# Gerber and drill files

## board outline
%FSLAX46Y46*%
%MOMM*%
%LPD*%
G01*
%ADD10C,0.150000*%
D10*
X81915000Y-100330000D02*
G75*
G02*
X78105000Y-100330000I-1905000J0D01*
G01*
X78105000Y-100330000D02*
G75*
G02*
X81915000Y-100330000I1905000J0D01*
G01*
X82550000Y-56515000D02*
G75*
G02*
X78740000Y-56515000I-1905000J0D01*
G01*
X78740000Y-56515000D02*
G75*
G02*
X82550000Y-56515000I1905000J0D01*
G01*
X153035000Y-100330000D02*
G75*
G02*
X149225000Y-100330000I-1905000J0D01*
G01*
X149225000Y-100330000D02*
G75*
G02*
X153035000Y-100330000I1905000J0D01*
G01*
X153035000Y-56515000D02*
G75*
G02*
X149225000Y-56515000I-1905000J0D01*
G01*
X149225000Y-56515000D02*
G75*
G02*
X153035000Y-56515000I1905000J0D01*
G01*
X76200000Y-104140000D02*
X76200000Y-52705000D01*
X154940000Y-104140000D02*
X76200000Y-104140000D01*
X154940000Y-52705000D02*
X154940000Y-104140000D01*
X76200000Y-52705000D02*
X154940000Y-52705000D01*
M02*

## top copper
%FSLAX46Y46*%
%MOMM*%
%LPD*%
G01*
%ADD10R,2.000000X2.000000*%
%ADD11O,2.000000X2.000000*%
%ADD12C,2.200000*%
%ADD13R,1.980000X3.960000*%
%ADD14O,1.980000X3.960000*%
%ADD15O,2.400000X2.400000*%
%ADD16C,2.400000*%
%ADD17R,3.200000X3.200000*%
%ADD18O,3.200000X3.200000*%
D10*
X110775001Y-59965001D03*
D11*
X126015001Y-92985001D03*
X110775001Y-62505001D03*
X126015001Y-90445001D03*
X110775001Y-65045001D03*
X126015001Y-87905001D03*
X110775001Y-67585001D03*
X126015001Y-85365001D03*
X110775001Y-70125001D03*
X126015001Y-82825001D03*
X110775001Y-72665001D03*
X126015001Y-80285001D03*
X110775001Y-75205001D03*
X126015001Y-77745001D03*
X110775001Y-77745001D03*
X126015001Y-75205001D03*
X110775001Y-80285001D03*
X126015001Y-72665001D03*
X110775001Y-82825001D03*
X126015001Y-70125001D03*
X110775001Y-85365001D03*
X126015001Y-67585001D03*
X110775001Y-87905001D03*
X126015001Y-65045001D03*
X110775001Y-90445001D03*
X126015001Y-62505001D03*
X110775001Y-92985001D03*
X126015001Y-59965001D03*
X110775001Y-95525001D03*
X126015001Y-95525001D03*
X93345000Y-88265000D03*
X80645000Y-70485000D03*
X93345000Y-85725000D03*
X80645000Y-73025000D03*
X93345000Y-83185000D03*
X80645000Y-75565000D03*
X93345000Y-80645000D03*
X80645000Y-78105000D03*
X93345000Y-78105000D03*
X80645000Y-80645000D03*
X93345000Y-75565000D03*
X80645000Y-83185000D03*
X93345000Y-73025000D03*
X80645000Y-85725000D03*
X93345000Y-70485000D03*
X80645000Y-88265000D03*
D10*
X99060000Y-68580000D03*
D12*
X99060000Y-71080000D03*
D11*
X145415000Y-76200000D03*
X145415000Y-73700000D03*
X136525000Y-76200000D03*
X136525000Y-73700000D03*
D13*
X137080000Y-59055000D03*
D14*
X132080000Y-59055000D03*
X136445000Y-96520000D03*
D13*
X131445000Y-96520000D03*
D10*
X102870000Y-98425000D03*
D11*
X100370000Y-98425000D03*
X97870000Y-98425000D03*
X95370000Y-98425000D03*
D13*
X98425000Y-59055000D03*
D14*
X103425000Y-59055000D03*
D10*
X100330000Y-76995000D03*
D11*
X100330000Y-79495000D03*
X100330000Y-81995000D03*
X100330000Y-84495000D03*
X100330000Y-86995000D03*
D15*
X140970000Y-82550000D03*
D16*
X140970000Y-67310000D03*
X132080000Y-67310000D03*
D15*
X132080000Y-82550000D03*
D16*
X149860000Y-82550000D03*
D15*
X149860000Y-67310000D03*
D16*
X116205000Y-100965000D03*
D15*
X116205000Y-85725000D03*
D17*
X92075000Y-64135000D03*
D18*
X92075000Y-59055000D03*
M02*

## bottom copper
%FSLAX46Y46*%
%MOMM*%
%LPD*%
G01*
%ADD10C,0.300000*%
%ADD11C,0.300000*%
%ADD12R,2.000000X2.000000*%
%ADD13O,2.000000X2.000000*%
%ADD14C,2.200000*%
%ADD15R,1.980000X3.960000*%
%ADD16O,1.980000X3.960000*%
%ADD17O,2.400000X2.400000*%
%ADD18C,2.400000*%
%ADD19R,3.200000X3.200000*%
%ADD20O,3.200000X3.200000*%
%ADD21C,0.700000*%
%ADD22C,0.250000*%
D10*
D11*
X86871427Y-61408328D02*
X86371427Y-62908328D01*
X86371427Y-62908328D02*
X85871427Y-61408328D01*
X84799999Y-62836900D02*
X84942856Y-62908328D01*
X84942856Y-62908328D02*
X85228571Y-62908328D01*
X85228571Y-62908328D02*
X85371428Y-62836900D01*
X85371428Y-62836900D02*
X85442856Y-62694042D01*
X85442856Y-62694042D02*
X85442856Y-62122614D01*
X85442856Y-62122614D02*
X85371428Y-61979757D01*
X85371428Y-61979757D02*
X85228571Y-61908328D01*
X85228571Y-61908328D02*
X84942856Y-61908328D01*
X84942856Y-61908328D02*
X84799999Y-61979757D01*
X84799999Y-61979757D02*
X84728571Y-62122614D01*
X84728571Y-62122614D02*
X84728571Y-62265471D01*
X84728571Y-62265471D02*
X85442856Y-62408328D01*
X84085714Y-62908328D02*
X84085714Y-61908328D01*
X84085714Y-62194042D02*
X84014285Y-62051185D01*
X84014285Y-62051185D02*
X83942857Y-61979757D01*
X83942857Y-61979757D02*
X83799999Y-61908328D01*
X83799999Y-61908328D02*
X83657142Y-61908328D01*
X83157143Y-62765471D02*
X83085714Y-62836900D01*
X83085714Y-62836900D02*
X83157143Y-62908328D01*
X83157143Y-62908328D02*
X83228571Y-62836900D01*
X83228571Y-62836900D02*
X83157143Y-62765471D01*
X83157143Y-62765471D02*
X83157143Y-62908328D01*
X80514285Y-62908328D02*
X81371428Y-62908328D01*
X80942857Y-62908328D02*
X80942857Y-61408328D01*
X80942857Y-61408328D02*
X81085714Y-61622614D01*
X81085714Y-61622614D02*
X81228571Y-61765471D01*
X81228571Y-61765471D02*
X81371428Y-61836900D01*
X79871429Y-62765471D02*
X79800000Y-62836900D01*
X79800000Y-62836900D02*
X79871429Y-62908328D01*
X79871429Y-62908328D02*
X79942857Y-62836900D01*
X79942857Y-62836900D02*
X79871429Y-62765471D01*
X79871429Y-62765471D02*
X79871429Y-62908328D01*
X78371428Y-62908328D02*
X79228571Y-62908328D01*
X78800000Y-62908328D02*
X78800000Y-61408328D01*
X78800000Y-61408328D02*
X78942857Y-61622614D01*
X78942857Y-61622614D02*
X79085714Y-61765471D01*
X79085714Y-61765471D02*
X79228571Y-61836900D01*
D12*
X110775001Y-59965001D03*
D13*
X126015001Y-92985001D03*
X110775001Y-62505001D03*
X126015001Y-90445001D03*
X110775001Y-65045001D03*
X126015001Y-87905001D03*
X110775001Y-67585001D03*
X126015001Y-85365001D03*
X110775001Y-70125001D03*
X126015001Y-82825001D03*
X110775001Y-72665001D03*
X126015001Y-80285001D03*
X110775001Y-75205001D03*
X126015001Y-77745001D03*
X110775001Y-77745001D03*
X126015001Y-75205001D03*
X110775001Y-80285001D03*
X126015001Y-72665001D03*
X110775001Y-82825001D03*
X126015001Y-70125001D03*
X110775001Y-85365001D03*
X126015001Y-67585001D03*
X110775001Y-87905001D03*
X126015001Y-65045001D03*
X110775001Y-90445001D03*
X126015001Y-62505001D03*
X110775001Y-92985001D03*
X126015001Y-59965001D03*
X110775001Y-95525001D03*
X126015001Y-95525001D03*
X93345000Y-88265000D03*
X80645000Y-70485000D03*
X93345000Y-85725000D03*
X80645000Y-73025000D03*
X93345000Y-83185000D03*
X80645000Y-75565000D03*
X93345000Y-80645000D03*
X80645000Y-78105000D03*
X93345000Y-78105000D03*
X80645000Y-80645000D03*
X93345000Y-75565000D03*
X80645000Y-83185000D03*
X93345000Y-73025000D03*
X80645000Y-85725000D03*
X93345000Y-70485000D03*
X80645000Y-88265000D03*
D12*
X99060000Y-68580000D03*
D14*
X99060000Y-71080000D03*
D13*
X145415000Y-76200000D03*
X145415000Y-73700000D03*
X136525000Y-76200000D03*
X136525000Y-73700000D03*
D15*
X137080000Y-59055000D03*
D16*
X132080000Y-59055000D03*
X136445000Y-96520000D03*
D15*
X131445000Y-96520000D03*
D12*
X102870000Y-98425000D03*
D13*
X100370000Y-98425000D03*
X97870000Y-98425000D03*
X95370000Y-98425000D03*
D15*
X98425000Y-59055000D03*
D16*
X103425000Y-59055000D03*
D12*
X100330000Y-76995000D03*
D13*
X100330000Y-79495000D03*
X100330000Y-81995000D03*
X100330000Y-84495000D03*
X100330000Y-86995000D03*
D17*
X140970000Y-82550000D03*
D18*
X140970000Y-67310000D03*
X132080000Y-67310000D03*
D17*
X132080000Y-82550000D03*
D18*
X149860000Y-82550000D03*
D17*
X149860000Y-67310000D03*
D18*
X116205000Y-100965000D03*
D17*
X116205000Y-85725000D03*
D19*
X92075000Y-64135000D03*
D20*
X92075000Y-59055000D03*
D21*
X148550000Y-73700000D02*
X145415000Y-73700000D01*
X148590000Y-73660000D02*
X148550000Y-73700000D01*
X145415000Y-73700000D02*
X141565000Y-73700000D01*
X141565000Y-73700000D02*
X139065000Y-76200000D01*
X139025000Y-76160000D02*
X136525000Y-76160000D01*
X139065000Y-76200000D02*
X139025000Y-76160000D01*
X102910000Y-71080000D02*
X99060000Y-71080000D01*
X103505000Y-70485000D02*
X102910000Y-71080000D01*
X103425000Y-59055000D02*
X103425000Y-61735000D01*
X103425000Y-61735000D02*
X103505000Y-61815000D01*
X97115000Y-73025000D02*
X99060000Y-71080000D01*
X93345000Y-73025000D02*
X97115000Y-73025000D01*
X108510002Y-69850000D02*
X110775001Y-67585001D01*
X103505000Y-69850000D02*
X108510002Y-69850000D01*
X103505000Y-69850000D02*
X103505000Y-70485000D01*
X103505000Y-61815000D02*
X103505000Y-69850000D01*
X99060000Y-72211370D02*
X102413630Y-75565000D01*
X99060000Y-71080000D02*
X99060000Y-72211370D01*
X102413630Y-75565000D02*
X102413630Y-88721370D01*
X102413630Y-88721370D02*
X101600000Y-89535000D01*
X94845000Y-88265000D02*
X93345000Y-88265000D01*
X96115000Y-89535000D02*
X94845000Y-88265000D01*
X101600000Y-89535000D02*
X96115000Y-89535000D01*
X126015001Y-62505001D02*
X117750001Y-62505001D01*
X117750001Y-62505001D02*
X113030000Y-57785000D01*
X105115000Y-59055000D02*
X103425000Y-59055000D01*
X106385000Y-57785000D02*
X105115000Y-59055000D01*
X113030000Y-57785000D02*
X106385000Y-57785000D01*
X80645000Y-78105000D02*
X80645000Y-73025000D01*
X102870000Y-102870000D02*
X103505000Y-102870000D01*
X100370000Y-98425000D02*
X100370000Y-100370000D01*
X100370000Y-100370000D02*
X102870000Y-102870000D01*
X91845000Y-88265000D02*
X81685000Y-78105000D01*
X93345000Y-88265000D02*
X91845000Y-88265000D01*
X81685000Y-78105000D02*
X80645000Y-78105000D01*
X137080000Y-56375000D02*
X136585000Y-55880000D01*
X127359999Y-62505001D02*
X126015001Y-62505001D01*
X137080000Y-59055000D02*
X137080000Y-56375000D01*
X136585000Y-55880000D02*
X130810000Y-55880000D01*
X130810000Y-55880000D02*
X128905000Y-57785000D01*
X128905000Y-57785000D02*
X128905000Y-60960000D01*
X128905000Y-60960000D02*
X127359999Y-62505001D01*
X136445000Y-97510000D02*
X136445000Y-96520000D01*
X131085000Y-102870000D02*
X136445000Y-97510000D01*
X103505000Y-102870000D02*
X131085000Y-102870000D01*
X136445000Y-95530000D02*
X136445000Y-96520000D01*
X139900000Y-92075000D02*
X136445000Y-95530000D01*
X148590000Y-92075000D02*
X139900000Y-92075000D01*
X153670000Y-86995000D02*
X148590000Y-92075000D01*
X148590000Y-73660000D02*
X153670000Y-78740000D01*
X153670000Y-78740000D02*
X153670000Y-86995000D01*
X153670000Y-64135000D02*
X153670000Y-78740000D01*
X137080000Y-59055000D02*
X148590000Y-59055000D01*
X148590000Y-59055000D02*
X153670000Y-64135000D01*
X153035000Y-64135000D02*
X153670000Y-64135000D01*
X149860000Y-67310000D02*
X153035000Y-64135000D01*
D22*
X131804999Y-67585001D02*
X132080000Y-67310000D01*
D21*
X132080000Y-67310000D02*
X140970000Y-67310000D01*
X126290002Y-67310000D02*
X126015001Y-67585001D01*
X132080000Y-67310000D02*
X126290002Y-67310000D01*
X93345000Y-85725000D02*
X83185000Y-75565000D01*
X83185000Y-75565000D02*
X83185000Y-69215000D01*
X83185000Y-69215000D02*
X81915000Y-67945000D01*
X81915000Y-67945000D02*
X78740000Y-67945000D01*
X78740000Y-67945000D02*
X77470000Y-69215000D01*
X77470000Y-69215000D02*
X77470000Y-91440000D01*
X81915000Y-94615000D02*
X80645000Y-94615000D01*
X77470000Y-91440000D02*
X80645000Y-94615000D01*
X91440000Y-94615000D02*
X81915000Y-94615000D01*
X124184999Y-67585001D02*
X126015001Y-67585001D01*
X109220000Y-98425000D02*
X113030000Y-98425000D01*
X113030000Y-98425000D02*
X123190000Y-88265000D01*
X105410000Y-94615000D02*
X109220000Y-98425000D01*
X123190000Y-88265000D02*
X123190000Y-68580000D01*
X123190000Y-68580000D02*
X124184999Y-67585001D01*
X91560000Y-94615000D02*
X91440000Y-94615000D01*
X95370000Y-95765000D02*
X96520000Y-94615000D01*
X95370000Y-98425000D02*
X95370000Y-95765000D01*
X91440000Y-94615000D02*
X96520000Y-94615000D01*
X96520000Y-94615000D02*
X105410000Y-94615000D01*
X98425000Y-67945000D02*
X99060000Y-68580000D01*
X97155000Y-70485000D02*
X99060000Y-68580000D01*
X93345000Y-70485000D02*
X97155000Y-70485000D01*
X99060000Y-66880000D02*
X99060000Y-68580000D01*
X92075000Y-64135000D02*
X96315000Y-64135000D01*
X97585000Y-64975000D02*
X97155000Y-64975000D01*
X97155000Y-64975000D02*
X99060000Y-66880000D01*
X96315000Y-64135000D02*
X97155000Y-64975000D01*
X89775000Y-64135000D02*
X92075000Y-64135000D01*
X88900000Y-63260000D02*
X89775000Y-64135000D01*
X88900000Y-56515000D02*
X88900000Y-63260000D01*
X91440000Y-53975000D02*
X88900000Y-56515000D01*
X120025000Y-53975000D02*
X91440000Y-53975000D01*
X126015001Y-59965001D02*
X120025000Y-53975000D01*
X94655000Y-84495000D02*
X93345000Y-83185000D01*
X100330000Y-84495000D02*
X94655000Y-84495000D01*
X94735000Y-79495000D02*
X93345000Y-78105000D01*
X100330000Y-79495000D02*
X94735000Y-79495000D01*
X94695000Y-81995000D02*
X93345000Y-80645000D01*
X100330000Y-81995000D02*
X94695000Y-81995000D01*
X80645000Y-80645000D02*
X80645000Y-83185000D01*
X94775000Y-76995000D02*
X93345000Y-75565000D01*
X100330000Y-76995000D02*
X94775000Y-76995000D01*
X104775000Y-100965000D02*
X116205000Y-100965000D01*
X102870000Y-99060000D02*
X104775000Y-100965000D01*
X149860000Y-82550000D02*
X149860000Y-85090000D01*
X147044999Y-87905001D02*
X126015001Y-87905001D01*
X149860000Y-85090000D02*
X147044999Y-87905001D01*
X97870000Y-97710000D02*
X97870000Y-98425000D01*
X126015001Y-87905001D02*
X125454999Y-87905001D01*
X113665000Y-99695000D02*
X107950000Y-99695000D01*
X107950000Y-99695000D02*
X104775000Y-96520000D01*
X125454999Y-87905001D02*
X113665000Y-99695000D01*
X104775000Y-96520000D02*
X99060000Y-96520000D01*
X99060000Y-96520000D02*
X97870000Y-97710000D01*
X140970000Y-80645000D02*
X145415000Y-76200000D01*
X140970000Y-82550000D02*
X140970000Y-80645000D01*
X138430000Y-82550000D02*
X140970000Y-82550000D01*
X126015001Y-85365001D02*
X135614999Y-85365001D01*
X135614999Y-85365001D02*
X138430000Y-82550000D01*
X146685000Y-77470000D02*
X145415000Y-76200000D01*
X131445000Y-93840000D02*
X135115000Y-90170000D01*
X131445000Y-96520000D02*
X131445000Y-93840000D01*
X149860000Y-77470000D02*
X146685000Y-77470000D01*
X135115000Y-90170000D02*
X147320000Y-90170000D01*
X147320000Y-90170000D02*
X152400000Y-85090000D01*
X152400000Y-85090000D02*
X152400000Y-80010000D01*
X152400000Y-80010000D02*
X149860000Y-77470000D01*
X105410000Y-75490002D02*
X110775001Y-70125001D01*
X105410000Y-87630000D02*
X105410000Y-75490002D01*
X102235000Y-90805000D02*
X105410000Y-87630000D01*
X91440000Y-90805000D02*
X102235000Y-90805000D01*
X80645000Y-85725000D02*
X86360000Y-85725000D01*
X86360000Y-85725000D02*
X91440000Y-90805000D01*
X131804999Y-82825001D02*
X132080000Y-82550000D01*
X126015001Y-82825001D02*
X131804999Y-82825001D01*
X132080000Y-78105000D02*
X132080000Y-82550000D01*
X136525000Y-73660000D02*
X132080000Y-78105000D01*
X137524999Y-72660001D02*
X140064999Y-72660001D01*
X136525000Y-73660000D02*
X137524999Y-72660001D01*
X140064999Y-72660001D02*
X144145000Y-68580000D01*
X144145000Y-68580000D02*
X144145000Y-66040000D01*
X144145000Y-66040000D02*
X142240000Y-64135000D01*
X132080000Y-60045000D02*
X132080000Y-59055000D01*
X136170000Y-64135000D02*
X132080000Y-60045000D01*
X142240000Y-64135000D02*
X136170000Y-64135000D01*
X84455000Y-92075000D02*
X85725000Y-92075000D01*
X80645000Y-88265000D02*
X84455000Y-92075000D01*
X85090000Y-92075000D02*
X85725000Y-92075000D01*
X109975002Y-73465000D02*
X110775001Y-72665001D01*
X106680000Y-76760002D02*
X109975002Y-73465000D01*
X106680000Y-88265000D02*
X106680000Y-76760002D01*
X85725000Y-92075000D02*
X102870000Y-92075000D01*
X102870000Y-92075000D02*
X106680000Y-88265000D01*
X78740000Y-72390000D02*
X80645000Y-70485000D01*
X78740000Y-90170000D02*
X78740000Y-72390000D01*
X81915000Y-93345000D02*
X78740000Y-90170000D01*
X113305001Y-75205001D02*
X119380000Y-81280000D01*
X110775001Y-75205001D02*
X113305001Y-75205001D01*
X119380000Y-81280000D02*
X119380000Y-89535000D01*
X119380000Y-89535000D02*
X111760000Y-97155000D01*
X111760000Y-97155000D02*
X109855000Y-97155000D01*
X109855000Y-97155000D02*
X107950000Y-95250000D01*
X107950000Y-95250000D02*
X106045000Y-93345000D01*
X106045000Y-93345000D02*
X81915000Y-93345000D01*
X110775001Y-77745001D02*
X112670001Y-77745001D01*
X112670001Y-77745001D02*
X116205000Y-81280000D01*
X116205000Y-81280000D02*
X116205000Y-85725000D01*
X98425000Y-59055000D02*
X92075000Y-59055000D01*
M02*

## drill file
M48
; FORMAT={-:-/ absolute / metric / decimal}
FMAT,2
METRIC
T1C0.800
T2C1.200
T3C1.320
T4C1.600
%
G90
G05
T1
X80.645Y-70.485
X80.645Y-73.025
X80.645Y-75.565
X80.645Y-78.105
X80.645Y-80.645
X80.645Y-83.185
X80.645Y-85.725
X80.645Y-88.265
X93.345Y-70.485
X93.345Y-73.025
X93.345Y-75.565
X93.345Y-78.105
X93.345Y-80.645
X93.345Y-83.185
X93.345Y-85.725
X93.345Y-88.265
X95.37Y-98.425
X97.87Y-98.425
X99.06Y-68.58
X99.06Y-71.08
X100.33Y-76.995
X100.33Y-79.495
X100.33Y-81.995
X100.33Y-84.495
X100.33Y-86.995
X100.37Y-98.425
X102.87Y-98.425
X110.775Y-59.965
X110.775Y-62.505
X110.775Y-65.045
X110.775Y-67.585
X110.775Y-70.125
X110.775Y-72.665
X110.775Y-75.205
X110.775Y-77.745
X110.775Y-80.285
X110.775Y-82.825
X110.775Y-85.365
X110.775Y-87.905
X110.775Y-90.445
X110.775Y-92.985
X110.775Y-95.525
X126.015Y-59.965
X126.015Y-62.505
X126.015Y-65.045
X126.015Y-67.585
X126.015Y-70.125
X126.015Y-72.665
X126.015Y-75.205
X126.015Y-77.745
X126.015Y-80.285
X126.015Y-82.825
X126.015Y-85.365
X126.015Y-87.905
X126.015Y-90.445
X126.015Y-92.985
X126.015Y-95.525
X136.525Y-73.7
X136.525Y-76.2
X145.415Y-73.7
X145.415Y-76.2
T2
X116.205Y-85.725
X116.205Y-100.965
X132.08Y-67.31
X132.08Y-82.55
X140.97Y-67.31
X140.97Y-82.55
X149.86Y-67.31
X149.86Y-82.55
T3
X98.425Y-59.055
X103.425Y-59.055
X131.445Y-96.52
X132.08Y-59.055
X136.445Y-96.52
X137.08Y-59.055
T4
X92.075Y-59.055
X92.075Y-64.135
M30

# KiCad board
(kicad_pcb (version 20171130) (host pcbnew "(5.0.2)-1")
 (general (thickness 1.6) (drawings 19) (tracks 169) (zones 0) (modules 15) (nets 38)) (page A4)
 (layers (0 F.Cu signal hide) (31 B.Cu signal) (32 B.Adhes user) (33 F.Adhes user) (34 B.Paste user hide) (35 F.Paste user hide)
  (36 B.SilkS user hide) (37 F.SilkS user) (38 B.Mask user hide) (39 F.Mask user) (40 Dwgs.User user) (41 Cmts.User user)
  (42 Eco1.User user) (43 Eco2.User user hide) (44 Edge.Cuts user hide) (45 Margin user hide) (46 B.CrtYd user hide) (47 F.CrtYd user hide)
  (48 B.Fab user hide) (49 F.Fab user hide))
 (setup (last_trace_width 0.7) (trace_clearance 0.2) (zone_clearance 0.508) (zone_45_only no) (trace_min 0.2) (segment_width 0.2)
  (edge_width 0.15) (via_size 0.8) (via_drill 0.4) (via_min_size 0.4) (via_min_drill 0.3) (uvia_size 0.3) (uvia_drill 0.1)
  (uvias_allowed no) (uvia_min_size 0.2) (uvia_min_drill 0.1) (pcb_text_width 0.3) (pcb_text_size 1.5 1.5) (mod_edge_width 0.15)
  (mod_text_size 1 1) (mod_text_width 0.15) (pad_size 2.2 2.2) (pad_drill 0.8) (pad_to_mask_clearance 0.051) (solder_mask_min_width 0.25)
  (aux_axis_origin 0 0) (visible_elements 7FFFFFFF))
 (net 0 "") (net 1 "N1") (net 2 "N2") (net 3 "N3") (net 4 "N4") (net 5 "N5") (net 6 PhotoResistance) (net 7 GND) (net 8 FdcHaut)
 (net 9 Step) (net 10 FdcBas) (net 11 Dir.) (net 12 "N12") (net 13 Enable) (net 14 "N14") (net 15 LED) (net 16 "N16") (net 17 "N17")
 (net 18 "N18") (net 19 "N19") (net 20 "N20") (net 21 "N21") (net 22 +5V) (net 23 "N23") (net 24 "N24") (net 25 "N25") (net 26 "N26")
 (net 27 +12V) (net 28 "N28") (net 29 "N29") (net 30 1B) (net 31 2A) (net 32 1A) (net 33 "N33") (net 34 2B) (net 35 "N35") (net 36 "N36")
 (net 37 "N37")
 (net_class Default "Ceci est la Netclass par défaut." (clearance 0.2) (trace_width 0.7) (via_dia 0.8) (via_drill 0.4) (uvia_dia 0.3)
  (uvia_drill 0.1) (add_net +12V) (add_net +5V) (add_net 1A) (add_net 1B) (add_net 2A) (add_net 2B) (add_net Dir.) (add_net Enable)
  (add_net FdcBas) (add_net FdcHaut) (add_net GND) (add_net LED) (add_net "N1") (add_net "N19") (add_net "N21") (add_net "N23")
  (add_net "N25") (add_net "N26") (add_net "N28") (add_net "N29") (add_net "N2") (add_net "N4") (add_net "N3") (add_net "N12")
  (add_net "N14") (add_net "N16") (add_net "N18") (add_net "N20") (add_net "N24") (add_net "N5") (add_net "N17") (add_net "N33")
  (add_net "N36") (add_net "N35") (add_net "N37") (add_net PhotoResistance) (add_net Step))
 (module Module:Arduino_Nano (layer F.Cu) (at 110.775001 59.965001)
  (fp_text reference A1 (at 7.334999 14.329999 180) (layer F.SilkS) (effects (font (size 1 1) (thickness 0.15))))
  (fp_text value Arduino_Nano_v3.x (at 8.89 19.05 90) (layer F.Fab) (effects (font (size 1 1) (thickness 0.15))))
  (pad 1 thru_hole rect (at 0 0) (size 2 2) (drill 0.8) (layers *.Cu *.Mask) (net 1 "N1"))
  (pad 17 thru_hole oval (at 15.24 33.02) (size 2 2) (drill 0.8) (layers *.Cu *.Mask) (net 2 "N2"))
  (pad 2 thru_hole oval (at 0 2.54) (size 2 2) (drill 0.8) (layers *.Cu *.Mask) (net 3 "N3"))
  (pad 18 thru_hole oval (at 15.24 30.48) (size 2 2) (drill 0.8) (layers *.Cu *.Mask) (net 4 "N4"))
  (pad 3 thru_hole oval (at 0 5.08) (size 2 2) (drill 0.8) (layers *.Cu *.Mask) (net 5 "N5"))
  (pad 19 thru_hole oval (at 15.24 27.94) (size 2 2) (drill 0.8) (layers *.Cu *.Mask) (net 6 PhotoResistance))
  (pad 4 thru_hole oval (at 0 7.62) (size 2 2) (drill 0.8) (layers *.Cu *.Mask) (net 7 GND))
  (pad 20 thru_hole oval (at 15.24 25.4) (size 2 2) (drill 0.8) (layers *.Cu *.Mask) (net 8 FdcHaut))
  (pad 5 thru_hole oval (at 0 10.16) (size 2 2) (drill 0.8) (layers *.Cu *.Mask) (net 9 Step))
  (pad 21 thru_hole oval (at 15.24 22.86) (size 2 2) (drill 0.8) (layers *.Cu *.Mask) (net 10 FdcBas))
  (pad 6 thru_hole oval (at 0 12.7) (size 2 2) (drill 0.8) (layers *.Cu *.Mask) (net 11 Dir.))
  (pad 22 thru_hole oval (at 15.24 20.32) (size 2 2) (drill 0.8) (layers *.Cu *.Mask) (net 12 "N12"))
  (pad 7 thru_hole oval (at 0 15.24) (size 2 2) (drill 0.8) (layers *.Cu *.Mask) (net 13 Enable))
  (pad 23 thru_hole oval (at 15.24 17.78) (size 2 2) (drill 0.8) (layers *.Cu *.Mask) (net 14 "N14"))
  (pad 8 thru_hole oval (at 0 17.78) (size 2 2) (drill 0.8) (layers *.Cu *.Mask) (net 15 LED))
  (pad 24 thru_hole oval (at 15.24 15.24) (size 2 2) (drill 0.8) (layers *.Cu *.Mask) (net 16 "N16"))
  (pad 9 thru_hole oval (at 0 20.32) (size 2 2) (drill 0.8) (layers *.Cu *.Mask) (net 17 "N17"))
  (pad 25 thru_hole oval (at 15.24 12.7) (size 2 2) (drill 0.8) (layers *.Cu *.Mask) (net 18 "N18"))
  (pad 10 thru_hole oval (at 0 22.86) (size 2 2) (drill 0.8) (layers *.Cu *.Mask) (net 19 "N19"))
  (pad 26 thru_hole oval (at 15.24 10.16) (size 2 2) (drill 0.8) (layers *.Cu *.Mask) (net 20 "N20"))
  (pad 11 thru_hole oval (at 0 25.4) (size 2 2) (drill 0.8) (layers *.Cu *.Mask) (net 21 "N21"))
  (pad 27 thru_hole oval (at 15.24 7.62) (size 2 2) (drill 0.8) (layers *.Cu *.Mask) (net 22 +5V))
  (pad 12 thru_hole oval (at 0 27.94) (size 2 2) (drill 0.8) (layers *.Cu *.Mask) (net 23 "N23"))
  (pad 28 thru_hole oval (at 15.24 5.08) (size 2 2) (drill 0.8) (layers *.Cu *.Mask) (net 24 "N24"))
  (pad 13 thru_hole oval (at 0 30.48) (size 2 2) (drill 0.8) (layers *.Cu *.Mask) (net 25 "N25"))
  (pad 29 thru_hole oval (at 15.24 2.54) (size 2 2) (drill 0.8) (layers *.Cu *.Mask) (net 7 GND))
  (pad 14 thru_hole oval (at 0 33.02) (size 2 2) (drill 0.8) (layers *.Cu *.Mask) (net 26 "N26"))
  (pad 30 thru_hole oval (at 15.24 0) (size 2 2) (drill 0.8) (layers *.Cu *.Mask) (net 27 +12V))
  (pad 15 thru_hole oval (at 0 35.56) (size 2 2) (drill 0.8) (layers *.Cu *.Mask) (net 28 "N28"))
  (pad 16 thru_hole oval (at 15.24 35.56) (size 2 2) (drill 0.8) (layers *.Cu *.Mask) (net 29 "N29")))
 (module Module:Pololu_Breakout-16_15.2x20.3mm (layer F.Cu) (at 93.345 88.265 180)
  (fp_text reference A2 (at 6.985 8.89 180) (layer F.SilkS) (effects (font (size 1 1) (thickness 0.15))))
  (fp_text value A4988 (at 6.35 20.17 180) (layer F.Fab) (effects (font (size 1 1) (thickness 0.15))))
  (pad 1 thru_hole oval (at 0 0 180) (size 2 2) (drill 0.8) (layers *.Cu *.Mask) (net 7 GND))
  (pad 9 thru_hole oval (at 12.7 17.78 180) (size 2 2) (drill 0.8) (layers *.Cu *.Mask) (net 13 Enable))
  (pad 2 thru_hole oval (at 0 2.54 180) (size 2 2) (drill 0.8) (layers *.Cu *.Mask) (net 22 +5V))
  (pad 10 thru_hole oval (at 12.7 15.24 180) (size 2 2) (drill 0.8) (layers *.Cu *.Mask) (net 7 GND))
  (pad 3 thru_hole oval (at 0 5.08 180) (size 2 2) (drill 0.8) (layers *.Cu *.Mask) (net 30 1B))
  (pad 11 thru_hole oval (at 12.7 12.7 180) (size 2 2) (drill 0.8) (layers *.Cu *.Mask) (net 7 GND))
  (pad 4 thru_hole oval (at 0 7.62 180) (size 2 2) (drill 0.8) (layers *.Cu *.Mask) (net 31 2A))
  (pad 12 thru_hole oval (at 12.7 10.16 180) (size 2 2) (drill 0.8) (layers *.Cu *.Mask) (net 7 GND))
  (pad 5 thru_hole oval (at 0 10.16 180) (size 2 2) (drill 0.8) (layers *.Cu *.Mask) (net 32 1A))
  (pad 13 thru_hole oval (at 12.7 7.62 180) (size 2 2) (drill 0.8) (layers *.Cu *.Mask) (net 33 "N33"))
  (pad 6 thru_hole oval (at 0 12.7 180) (size 2 2) (drill 0.8) (layers *.Cu *.Mask) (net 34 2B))
  (pad 14 thru_hole oval (at 12.7 5.08 180) (size 2 2) (drill 0.8) (layers *.Cu *.Mask) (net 33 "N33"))
  (pad 7 thru_hole oval (at 0 15.24 180) (size 2 2) (drill 0.8) (layers *.Cu *.Mask) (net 7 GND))
  (pad 15 thru_hole oval (at 12.7 2.54 180) (size 2 2) (drill 0.8) (layers *.Cu *.Mask) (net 9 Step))
  (pad 8 thru_hole oval (at 0 17.78 180) (size 2 2) (drill 0.8) (layers *.Cu *.Mask) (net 27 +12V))
  (pad 16 thru_hole oval (at 12.7 0 180) (size 2 2) (drill 0.8) (layers *.Cu *.Mask) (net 11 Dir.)))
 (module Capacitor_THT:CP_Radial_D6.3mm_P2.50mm (layer F.Cu) (at 99.06 68.58 270)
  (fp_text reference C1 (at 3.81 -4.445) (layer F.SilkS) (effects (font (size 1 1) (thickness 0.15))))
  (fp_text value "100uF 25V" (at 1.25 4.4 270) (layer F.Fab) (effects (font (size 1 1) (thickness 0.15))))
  (pad 1 thru_hole rect (at 0 0 270) (size 2 2) (drill 0.8) (layers *.Cu *.Mask) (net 27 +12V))
  (pad 2 thru_hole circle (at 2.5 0 270) (size 2.2 2.2) (drill 0.8) (layers *.Cu *.Mask) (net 7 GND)))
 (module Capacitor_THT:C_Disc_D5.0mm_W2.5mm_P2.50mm (layer F.Cu) (at 145.415 76.2 90)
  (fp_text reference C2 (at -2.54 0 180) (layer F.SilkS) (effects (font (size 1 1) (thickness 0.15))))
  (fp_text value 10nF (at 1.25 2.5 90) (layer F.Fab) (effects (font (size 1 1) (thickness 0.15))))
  (pad 1 thru_hole oval (at 0 0 90) (size 2 2) (drill 0.8) (layers *.Cu *.Mask) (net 8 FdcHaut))
  (pad 2 thru_hole oval (at 2.5 0 90) (size 2 2) (drill 0.8) (layers *.Cu *.Mask) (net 7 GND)))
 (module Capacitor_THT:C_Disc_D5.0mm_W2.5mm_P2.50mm (layer F.Cu) (at 136.525 73.7 270)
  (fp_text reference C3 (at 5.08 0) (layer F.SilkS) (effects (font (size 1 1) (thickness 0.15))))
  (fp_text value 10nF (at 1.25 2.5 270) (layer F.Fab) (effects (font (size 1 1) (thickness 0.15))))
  (pad 2 thru_hole oval (at 2.5 0 270) (size 2 2) (drill 0.8) (layers *.Cu *.Mask) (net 7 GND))
  (pad 1 thru_hole oval (at 0 0 270) (size 2 2) (drill 0.8) (layers *.Cu *.Mask) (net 10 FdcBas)))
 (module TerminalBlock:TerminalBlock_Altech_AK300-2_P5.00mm (layer F.Cu) (at 137.08 59.055 180)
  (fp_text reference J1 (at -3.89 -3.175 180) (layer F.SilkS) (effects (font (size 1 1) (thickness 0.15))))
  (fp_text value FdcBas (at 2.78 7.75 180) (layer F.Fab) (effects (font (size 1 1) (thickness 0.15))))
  (pad 1 thru_hole rect (at 0 0 180) (size 1.98 3.96) (drill 1.32) (layers *.Cu *.Mask) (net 7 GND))
  (pad 2 thru_hole oval (at 5 0 180) (size 1.98 3.96) (drill 1.32) (layers *.Cu *.Mask) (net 10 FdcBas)))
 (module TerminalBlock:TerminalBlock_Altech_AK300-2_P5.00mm (layer F.Cu) (at 131.445 96.52)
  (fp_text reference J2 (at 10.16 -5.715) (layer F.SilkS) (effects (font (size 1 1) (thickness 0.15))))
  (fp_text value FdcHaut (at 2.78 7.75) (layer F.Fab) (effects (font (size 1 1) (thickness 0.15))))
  (pad 2 thru_hole oval (at 5 0) (size 1.98 3.96) (drill 1.32) (layers *.Cu *.Mask) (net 7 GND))
  (pad 1 thru_hole rect (at 0 0) (size 1.98 3.96) (drill 1.32) (layers *.Cu *.Mask) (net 8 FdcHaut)))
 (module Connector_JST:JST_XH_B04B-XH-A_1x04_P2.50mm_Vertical (layer F.Cu) (at 102.87 98.425 180)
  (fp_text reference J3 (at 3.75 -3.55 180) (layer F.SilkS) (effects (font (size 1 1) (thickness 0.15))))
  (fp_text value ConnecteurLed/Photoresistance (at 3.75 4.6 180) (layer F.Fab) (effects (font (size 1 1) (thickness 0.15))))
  (pad 1 thru_hole rect (at 0 0 180) (size 2 2) (drill 0.8) (layers *.Cu *.Mask) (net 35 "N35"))
  (pad 2 thru_hole oval (at 2.5 0 180) (size 2 2) (drill 0.8) (layers *.Cu *.Mask) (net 7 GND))
  (pad 3 thru_hole oval (at 5 0 180) (size 2 2) (drill 0.8) (layers *.Cu *.Mask) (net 6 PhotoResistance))
  (pad 4 thru_hole oval (at 7.5 0 180) (size 2 2) (drill 0.8) (layers *.Cu *.Mask) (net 22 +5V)))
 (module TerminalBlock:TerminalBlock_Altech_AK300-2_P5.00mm (layer F.Cu) (at 98.425 59.055)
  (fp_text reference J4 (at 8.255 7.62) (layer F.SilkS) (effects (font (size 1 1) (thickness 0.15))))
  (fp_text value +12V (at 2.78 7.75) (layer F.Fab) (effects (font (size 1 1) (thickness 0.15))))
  (pad 1 thru_hole rect (at 0 0) (size 1.98 3.96) (drill 1.32) (layers *.Cu *.Mask) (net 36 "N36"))
  (pad 2 thru_hole oval (at 5 0) (size 1.98 3.96) (drill 1.32) (layers *.Cu *.Mask) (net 7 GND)))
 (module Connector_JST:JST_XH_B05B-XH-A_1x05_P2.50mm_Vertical (layer F.Cu) (at 100.33 76.995 270)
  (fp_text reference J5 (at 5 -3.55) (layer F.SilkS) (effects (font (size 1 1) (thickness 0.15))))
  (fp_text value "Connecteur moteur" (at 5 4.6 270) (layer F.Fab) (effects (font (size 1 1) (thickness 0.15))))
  (pad 1 thru_hole rect (at 0 0 270) (size 2 2) (drill 0.8) (layers *.Cu *.Mask) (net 34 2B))
  (pad 2 thru_hole oval (at 2.5 0 270) (size 2 2) (drill 0.8) (layers *.Cu *.Mask) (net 32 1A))
  (pad 3 thru_hole oval (at 5 0 270) (size 2 2) (drill 0.8) (layers *.Cu *.Mask) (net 31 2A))
  (pad 4 thru_hole oval (at 7.5 0 270) (size 2 2) (drill 0.8) (layers *.Cu *.Mask) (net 30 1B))
  (pad 5 thru_hole oval (at 10 0 270) (size 2 2) (drill 0.8) (layers *.Cu *.Mask) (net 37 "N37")))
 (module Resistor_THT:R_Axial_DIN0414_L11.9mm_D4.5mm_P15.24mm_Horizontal (layer F.Cu) (at 140.97 67.31 270)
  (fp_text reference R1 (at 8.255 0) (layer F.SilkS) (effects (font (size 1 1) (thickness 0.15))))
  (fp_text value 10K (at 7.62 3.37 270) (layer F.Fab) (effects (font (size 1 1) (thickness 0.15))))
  (pad 2 thru_hole oval (at 15.24 0 270) (size 2.4 2.4) (drill 1.2) (layers *.Cu *.Mask) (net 8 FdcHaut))
  (pad 1 thru_hole circle (at 0 0 270) (size 2.4 2.4) (drill 1.2) (layers *.Cu *.Mask) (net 22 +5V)))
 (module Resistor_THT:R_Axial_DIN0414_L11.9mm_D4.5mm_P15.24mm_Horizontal (layer F.Cu) (at 132.08 67.31 270)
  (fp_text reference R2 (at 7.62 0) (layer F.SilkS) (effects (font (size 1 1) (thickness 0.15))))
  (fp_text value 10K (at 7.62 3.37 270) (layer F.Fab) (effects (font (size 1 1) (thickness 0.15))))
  (pad 1 thru_hole circle (at 0 0 270) (size 2.4 2.4) (drill 1.2) (layers *.Cu *.Mask) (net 22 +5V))
  (pad 2 thru_hole oval (at 15.24 0 270) (size 2.4 2.4) (drill 1.2) (layers *.Cu *.Mask) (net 10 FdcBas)))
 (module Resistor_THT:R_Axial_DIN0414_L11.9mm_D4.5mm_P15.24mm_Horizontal (layer F.Cu) (at 149.86 82.55 90)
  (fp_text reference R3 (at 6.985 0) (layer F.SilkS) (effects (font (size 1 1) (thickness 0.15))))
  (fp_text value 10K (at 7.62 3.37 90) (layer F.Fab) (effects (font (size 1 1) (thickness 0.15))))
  (pad 1 thru_hole circle (at 0 0 90) (size 2.4 2.4) (drill 1.2) (layers *.Cu *.Mask) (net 6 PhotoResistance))
  (pad 2 thru_hole oval (at 15.24 0 90) (size 2.4 2.4) (drill 1.2) (layers *.Cu *.Mask) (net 7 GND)))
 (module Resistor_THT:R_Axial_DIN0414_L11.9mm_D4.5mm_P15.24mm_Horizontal (layer F.Cu) (at 116.205 100.965 90)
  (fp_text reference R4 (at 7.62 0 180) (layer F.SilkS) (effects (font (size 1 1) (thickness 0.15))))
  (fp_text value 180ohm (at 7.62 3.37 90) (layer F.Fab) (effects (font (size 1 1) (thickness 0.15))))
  (pad 1 thru_hole circle (at 0 0 90) (size 2.4 2.4) (drill 1.2) (layers *.Cu *.Mask) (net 35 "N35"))
  (pad 2 thru_hole oval (at 15.24 0 90) (size 2.4 2.4) (drill 1.2) (layers *.Cu *.Mask) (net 15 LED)))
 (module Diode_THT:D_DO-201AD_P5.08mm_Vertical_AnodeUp (layer F.Cu) (at 92.075 64.135 90)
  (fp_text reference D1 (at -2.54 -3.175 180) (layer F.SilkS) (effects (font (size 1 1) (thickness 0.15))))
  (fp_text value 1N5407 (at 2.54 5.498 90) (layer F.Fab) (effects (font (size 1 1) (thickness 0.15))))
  (pad 1 thru_hole rect (at 0 0 90) (size 3.2 3.2) (drill 1.6) (layers *.Cu *.Mask) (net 27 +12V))
  (pad 2 thru_hole oval (at 5.08 0 90) (size 3.2 3.2) (drill 1.6) (layers *.Cu *.Mask) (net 36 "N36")))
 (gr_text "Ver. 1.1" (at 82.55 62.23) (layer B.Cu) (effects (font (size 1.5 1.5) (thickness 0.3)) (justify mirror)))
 (gr_circle (center 80.01 100.33) (end 81.915 100.33) (layer Edge.Cuts) (width 0.15))
 (gr_circle (center 80.645 56.515) (end 82.55 56.515) (layer Edge.Cuts) (width 0.15))
 (gr_circle (center 151.13 100.33) (end 151.13 98.425) (layer Edge.Cuts) (width 0.15))
 (gr_circle (center 151.13 56.515) (end 151.13 54.61) (layer Edge.Cuts) (width 0.15))
 (gr_line (start 76.2 104.14) (end 76.2 52.705) (layer Edge.Cuts) (width 0.15))
 (gr_line (start 154.94 104.14) (end 76.2 104.14) (layer Edge.Cuts) (width 0.15))
 (gr_line (start 154.94 52.705) (end 154.94 104.14) (layer Edge.Cuts) (width 0.15))
 (gr_line (start 76.2 52.705) (end 154.94 52.705) (layer Edge.Cuts) (width 0.15))
 (segment (start 148.55 73.7) (end 145.415 73.7) (width 0.7) (layer B.Cu) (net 7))
 (segment (start 148.59 73.66) (end 148.55 73.7) (width 0.7) (layer B.Cu) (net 7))
 (segment (start 145.415 73.7) (end 141.565 73.7) (width 0.7) (layer B.Cu) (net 7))
 (segment (start 141.565 73.7) (end 139.065 76.2) (width 0.7) (layer B.Cu) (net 7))
 (segment (start 139.025 76.16) (end 136.525 76.16) (width 0.7) (layer B.Cu) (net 7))
 (segment (start 139.065 76.2) (end 139.025 76.16) (width 0.7) (layer B.Cu) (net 7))
 (segment (start 102.91 71.08) (end 99.06 71.08) (width 0.7) (layer B.Cu) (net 7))
 (segment (start 103.505 70.485) (end 102.91 71.08) (width 0.7) (layer B.Cu) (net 7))
 (segment (start 103.425 59.055) (end 103.425 61.735) (width 0.7) (layer B.Cu) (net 7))
 (segment (start 103.425 61.735) (end 103.505 61.815) (width 0.7) (layer B.Cu) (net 7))
 (segment (start 97.115 73.025) (end 99.06 71.08) (width 0.7) (layer B.Cu) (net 7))
 (segment (start 93.345 73.025) (end 97.115 73.025) (width 0.7) (layer B.Cu) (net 7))
 (segment (start 108.510002 69.85) (end 110.775001 67.585001) (width 0.7) (layer B.Cu) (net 7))
 (segment (start 103.505 69.85) (end 108.510002 69.85) (width 0.7) (layer B.Cu) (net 7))
 (segment (start 103.505 69.85) (end 103.505 70.485) (width 0.7) (layer B.Cu) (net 7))
 (segment (start 103.505 61.815) (end 103.505 69.85) (width 0.7) (layer B.Cu) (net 7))
 (segment (start 99.06 72.21137) (end 102.41363 75.565) (width 0.7) (layer B.Cu) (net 7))
 (segment (start 99.06 71.08) (end 99.06 72.21137) (width 0.7) (layer B.Cu) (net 7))
 (segment (start 102.41363 75.565) (end 102.41363 88.72137) (width 0.7) (layer B.Cu) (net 7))
 (segment (start 102.41363 88.72137) (end 101.6 89.535) (width 0.7) (layer B.Cu) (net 7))
 (segment (start 94.845 88.265) (end 93.345 88.265) (width 0.7) (layer B.Cu) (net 7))
 (segment (start 96.115 89.535) (end 94.845 88.265) (width 0.7) (layer B.Cu) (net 7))
 (segment (start 101.6 89.535) (end 96.115 89.535) (width 0.7) (layer B.Cu) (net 7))
 (segment (start 126.015001 62.505001) (end 117.750001 62.505001) (width 0.7) (layer B.Cu) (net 7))
 (segment (start 117.750001 62.505001) (end 113.03 57.785) (width 0.7) (layer B.Cu) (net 7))
 (segment (start 105.115 59.055) (end 103.425 59.055) (width 0.7) (layer B.Cu) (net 7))
 (segment (start 106.385 57.785) (end 105.115 59.055) (width 0.7) (layer B.Cu) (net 7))
 (segment (start 113.03 57.785) (end 106.385 57.785) (width 0.7) (layer B.Cu) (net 7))
 (segment (start 80.645 78.105) (end 80.645 73.025) (width 0.7) (layer B.Cu) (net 7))
 (segment (start 102.87 102.87) (end 103.505 102.87) (width 0.7) (layer B.Cu) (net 7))
 (segment (start 100.37 98.425) (end 100.37 100.37) (width 0.7) (layer B.Cu) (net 7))
 (segment (start 100.37 100.37) (end 102.87 102.87) (width 0.7) (layer B.Cu) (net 7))
 (segment (start 91.845 88.265) (end 81.685 78.105) (width 0.7) (layer B.Cu) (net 7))
 (segment (start 93.345 88.265) (end 91.845 88.265) (width 0.7) (layer B.Cu) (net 7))
 (segment (start 81.685 78.105) (end 80.645 78.105) (width 0.7) (layer B.Cu) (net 7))
 (segment (start 137.08 56.375) (end 136.585 55.88) (width 0.7) (layer B.Cu) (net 7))
 (segment (start 127.359999 62.505001) (end 126.015001 62.505001) (width 0.7) (layer B.Cu) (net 7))
 (segment (start 137.08 59.055) (end 137.08 56.375) (width 0.7) (layer B.Cu) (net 7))
 (segment (start 136.585 55.88) (end 130.81 55.88) (width 0.7) (layer B.Cu) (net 7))
 (segment (start 130.81 55.88) (end 128.905 57.785) (width 0.7) (layer B.Cu) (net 7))
 (segment (start 128.905 57.785) (end 128.905 60.96) (width 0.7) (layer B.Cu) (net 7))
 (segment (start 128.905 60.96) (end 127.359999 62.505001) (width 0.7) (layer B.Cu) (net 7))
 (segment (start 136.445 97.51) (end 136.445 96.52) (width 0.7) (layer B.Cu) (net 7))
 (segment (start 131.085 102.87) (end 136.445 97.51) (width 0.7) (layer B.Cu) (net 7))
 (segment (start 103.505 102.87) (end 131.085 102.87) (width 0.7) (layer B.Cu) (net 7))
 (segment (start 136.445 95.53) (end 136.445 96.52) (width 0.7) (layer B.Cu) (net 7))
 (segment (start 139.9 92.075) (end 136.445 95.53) (width 0.7) (layer B.Cu) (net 7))
 (segment (start 148.59 92.075) (end 139.9 92.075) (width 0.7) (layer B.Cu) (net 7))
 (segment (start 153.67 86.995) (end 148.59 92.075) (width 0.7) (layer B.Cu) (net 7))
 (segment (start 148.59 73.66) (end 153.67 78.74) (width 0.7) (layer B.Cu) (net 7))
 (segment (start 153.67 78.74) (end 153.67 86.995) (width 0.7) (layer B.Cu) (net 7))
 (segment (start 153.67 64.135) (end 153.67 78.74) (width 0.7) (layer B.Cu) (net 7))
 (segment (start 137.08 59.055) (end 148.59 59.055) (width 0.7) (layer B.Cu) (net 7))
 (segment (start 148.59 59.055) (end 153.67 64.135) (width 0.7) (layer B.Cu) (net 7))
 (segment (start 153.035 64.135) (end 153.67 64.135) (width 0.7) (layer B.Cu) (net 7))
 (segment (start 149.86 67.31) (end 153.035 64.135) (width 0.7) (layer B.Cu) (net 7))
 (segment (start 131.804999 67.585001) (end 132.08 67.31) (width 0.25) (layer B.Cu) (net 22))
 (segment (start 132.08 67.31) (end 140.97 67.31) (width 0.7) (layer B.Cu) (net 22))
 (segment (start 126.290002 67.31) (end 126.015001 67.585001) (width 0.7) (layer B.Cu) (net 22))
 (segment (start 132.08 67.31) (end 126.290002 67.31) (width 0.7) (layer B.Cu) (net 22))
 (segment (start 93.345 85.725) (end 83.185 75.565) (width 0.7) (layer B.Cu) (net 22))
 (segment (start 83.185 75.565) (end 83.185 69.215) (width 0.7) (layer B.Cu) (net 22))
 (segment (start 83.185 69.215) (end 81.915 67.945) (width 0.7) (layer B.Cu) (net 22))
 (segment (start 81.915 67.945) (end 78.74 67.945) (width 0.7) (layer B.Cu) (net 22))
 (segment (start 78.74 67.945) (end 77.47 69.215) (width 0.7) (layer B.Cu) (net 22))
 (segment (start 77.47 69.215) (end 77.47 91.44) (width 0.7) (layer B.Cu) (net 22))
 (segment (start 81.915 94.615) (end 80.645 94.615) (width 0.7) (layer B.Cu) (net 22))
 (segment (start 77.47 91.44) (end 80.645 94.615) (width 0.7) (layer B.Cu) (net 22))
 (segment (start 91.44 94.615) (end 81.915 94.615) (width 0.7) (layer B.Cu) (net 22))
 (segment (start 124.184999 67.585001) (end 126.015001 67.585001) (width 0.7) (layer B.Cu) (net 22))
 (segment (start 109.22 98.425) (end 113.03 98.425) (width 0.7) (layer B.Cu) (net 22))
 (segment (start 113.03 98.425) (end 123.19 88.265) (width 0.7) (layer B.Cu) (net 22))
 (segment (start 105.41 94.615) (end 109.22 98.425) (width 0.7) (layer B.Cu) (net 22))
 (segment (start 123.19 88.265) (end 123.19 68.58) (width 0.7) (layer B.Cu) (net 22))
 (segment (start 123.19 68.58) (end 124.184999 67.585001) (width 0.7) (layer B.Cu) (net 22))
 (segment (start 91.56 94.615) (end 91.44 94.615) (width 0.7) (layer B.Cu) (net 22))
 (segment (start 95.37 95.765) (end 96.52 94.615) (width 0.7) (layer B.Cu) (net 22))
 (segment (start 95.37 98.425) (end 95.37 95.765) (width 0.7) (layer B.Cu) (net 22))
 (segment (start 91.44 94.615) (end 96.52 94.615) (width 0.7) (layer B.Cu) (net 22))
 (segment (start 96.52 94.615) (end 105.41 94.615) (width 0.7) (layer B.Cu) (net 22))
 (segment (start 98.425 67.945) (end 99.06 68.58) (width 0.7) (layer B.Cu) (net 27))
 (segment (start 97.155 70.485) (end 99.06 68.58) (width 0.7) (layer B.Cu) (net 27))
 (segment (start 93.345 70.485) (end 97.155 70.485) (width 0.7) (layer B.Cu) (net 27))
 (segment (start 99.06 66.88) (end 99.06 68.58) (width 0.7) (layer B.Cu) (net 27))
 (segment (start 92.075 64.135) (end 96.315 64.135) (width 0.7) (layer B.Cu) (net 27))
 (segment (start 97.585 64.975) (end 97.155 64.975) (width 0.7) (layer B.Cu) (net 27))
 (segment (start 97.155 64.975) (end 99.06 66.88) (width 0.7) (layer B.Cu) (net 27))
 (segment (start 96.315 64.135) (end 97.155 64.975) (width 0.7) (layer B.Cu) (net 27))
 (segment (start 89.775 64.135) (end 92.075 64.135) (width 0.7) (layer B.Cu) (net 27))
 (segment (start 88.9 63.26) (end 89.775 64.135) (width 0.7) (layer B.Cu) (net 27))
 (segment (start 88.9 56.515) (end 88.9 63.26) (width 0.7) (layer B.Cu) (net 27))
 (segment (start 91.44 53.975) (end 88.9 56.515) (width 0.7) (layer B.Cu) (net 27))
 (segment (start 120.025 53.975) (end 91.44 53.975) (width 0.7) (layer B.Cu) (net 27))
 (segment (start 126.015001 59.965001) (end 120.025 53.975) (width 0.7) (layer B.Cu) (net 27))
 (segment (start 94.655 84.495) (end 93.345 83.185) (width 0.7) (layer B.Cu) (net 30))
 (segment (start 100.33 84.495) (end 94.655 84.495) (width 0.7) (layer B.Cu) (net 30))
 (segment (start 94.735 79.495) (end 93.345 78.105) (width 0.7) (layer B.Cu) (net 32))
 (segment (start 100.33 79.495) (end 94.735 79.495) (width 0.7) (layer B.Cu) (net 32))
 (segment (start 94.695 81.995) (end 93.345 80.645) (width 0.7) (layer B.Cu) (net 31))
 (segment (start 100.33 81.995) (end 94.695 81.995) (width 0.7) (layer B.Cu) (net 31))
 (segment (start 80.645 80.645) (end 80.645 83.185) (width 0.7) (layer B.Cu) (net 33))
 (segment (start 94.775 76.995) (end 93.345 75.565) (width 0.7) (layer B.Cu) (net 34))
 (segment (start 100.33 76.995) (end 94.775 76.995) (width 0.7) (layer B.Cu) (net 34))
 (segment (start 104.775 100.965) (end 116.205 100.965) (width 0.7) (layer B.Cu) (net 35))
 (segment (start 102.87 99.06) (end 104.775 100.965) (width 0.7) (layer B.Cu) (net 35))
 (segment (start 149.86 82.55) (end 149.86 85.09) (width 0.7) (layer B.Cu) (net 6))
 (segment (start 147.044999 87.905001) (end 126.015001 87.905001) (width 0.7) (layer B.Cu) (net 6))
 (segment (start 149.86 85.09) (end 147.044999 87.905001) (width 0.7) (layer B.Cu) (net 6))
 (segment (start 97.87 97.71) (end 97.87 98.425) (width 0.7) (layer B.Cu) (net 6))
 (segment (start 126.015001 87.905001) (end 125.454999 87.905001) (width 0.7) (layer B.Cu) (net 6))
 (segment (start 113.665 99.695) (end 107.95 99.695) (width 0.7) (layer B.Cu) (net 6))
 (segment (start 107.95 99.695) (end 104.775 96.52) (width 0.7) (layer B.Cu) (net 6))
 (segment (start 125.454999 87.905001) (end 113.665 99.695) (width 0.7) (layer B.Cu) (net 6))
 (segment (start 104.775 96.52) (end 99.06 96.52) (width 0.7) (layer B.Cu) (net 6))
 (segment (start 99.06 96.52) (end 97.87 97.71) (width 0.7) (layer B.Cu) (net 6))
 (segment (start 140.97 80.645) (end 145.415 76.2) (width 0.7) (layer B.Cu) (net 8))
 (segment (start 140.97 82.55) (end 140.97 80.645) (width 0.7) (layer B.Cu) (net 8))
 (segment (start 138.43 82.55) (end 140.97 82.55) (width 0.7) (layer B.Cu) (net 8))
 (segment (start 126.015001 85.365001) (end 135.614999 85.365001) (width 0.7) (layer B.Cu) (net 8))
 (segment (start 135.614999 85.365001) (end 138.43 82.55) (width 0.7) (layer B.Cu) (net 8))
 (segment (start 146.685 77.47) (end 145.415 76.2) (width 0.7) (layer B.Cu) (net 8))
 (segment (start 131.445 93.84) (end 135.115 90.17) (width 0.7) (layer B.Cu) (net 8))
 (segment (start 131.445 96.52) (end 131.445 93.84) (width 0.7) (layer B.Cu) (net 8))
 (segment (start 149.86 77.47) (end 146.685 77.47) (width 0.7) (layer B.Cu) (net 8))
 (segment (start 135.115 90.17) (end 147.32 90.17) (width 0.7) (layer B.Cu) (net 8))
 (segment (start 147.32 90.17) (end 152.4 85.09) (width 0.7) (layer B.Cu) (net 8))
 (segment (start 152.4 85.09) (end 152.4 80.01) (width 0.7) (layer B.Cu) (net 8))
 (segment (start 152.4 80.01) (end 149.86 77.47) (width 0.7) (layer B.Cu) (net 8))
 (segment (start 105.41 75.490002) (end 110.775001 70.125001) (width 0.7) (layer B.Cu) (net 9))
 (segment (start 105.41 87.63) (end 105.41 75.490002) (width 0.7) (layer B.Cu) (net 9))
 (segment (start 102.235 90.805) (end 105.41 87.63) (width 0.7) (layer B.Cu) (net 9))
 (segment (start 91.44 90.805) (end 102.235 90.805) (width 0.7) (layer B.Cu) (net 9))
 (segment (start 80.645 85.725) (end 86.36 85.725) (width 0.7) (layer B.Cu) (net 9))
 (segment (start 86.36 85.725) (end 91.44 90.805) (width 0.7) (layer B.Cu) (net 9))
 (segment (start 131.804999 82.825001) (end 132.08 82.55) (width 0.7) (layer B.Cu) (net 10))
 (segment (start 126.015001 82.825001) (end 131.804999 82.825001) (width 0.7) (layer B.Cu) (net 10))
 (segment (start 132.08 78.105) (end 132.08 82.55) (width 0.7) (layer B.Cu) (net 10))
 (segment (start 136.525 73.66) (end 132.08 78.105) (width 0.7) (layer B.Cu) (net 10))
 (segment (start 137.524999 72.660001) (end 140.064999 72.660001) (width 0.7) (layer B.Cu) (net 10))
 (segment (start 136.525 73.66) (end 137.524999 72.660001) (width 0.7) (layer B.Cu) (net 10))
 (segment (start 140.064999 72.660001) (end 144.145 68.58) (width 0.7) (layer B.Cu) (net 10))
 (segment (start 144.145 68.58) (end 144.145 66.04) (width 0.7) (layer B.Cu) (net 10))
 (segment (start 144.145 66.04) (end 142.24 64.135) (width 0.7) (layer B.Cu) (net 10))
 (segment (start 132.08 60.045) (end 132.08 59.055) (width 0.7) (layer B.Cu) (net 10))
 (segment (start 136.17 64.135) (end 132.08 60.045) (width 0.7) (layer B.Cu) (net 10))
 (segment (start 142.24 64.135) (end 136.17 64.135) (width 0.7) (layer B.Cu) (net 10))
 (segment (start 84.455 92.075) (end 85.725 92.075) (width 0.7) (layer B.Cu) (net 11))
 (segment (start 80.645 88.265) (end 84.455 92.075) (width 0.7) (layer B.Cu) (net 11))
 (segment (start 85.09 92.075) (end 85.725 92.075) (width 0.7) (layer B.Cu) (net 11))
 (segment (start 109.975002 73.465) (end 110.775001 72.665001) (width 0.7) (layer B.Cu) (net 11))
 (segment (start 106.68 76.760002) (end 109.975002 73.465) (width 0.7) (layer B.Cu) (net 11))
 (segment (start 106.68 88.265) (end 106.68 76.760002) (width 0.7) (layer B.Cu) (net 11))
 (segment (start 85.725 92.075) (end 102.87 92.075) (width 0.7) (layer B.Cu) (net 11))
 (segment (start 102.87 92.075) (end 106.68 88.265) (width 0.7) (layer B.Cu) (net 11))
 (segment (start 78.74 72.39) (end 80.645 70.485) (width 0.7) (layer B.Cu) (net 13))
 (segment (start 78.74 90.17) (end 78.74 72.39) (width 0.7) (layer B.Cu) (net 13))
 (segment (start 81.915 93.345) (end 78.74 90.17) (width 0.7) (layer B.Cu) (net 13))
 (segment (start 113.305001 75.205001) (end 119.38 81.28) (width 0.7) (layer B.Cu) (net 13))
 (segment (start 110.775001 75.205001) (end 113.305001 75.205001) (width 0.7) (layer B.Cu) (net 13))
 (segment (start 119.38 81.28) (end 119.38 89.535) (width 0.7) (layer B.Cu) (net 13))
 (segment (start 119.38 89.535) (end 111.76 97.155) (width 0.7) (layer B.Cu) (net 13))
 (segment (start 111.76 97.155) (end 109.855 97.155) (width 0.7) (layer B.Cu) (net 13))
 (segment (start 109.855 97.155) (end 107.95 95.25) (width 0.7) (layer B.Cu) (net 13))
 (segment (start 107.95 95.25) (end 106.045 93.345) (width 0.7) (layer B.Cu) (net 13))
 (segment (start 106.045 93.345) (end 81.915 93.345) (width 0.7) (layer B.Cu) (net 13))
 (segment (start 110.775001 77.745001) (end 112.670001 77.745001) (width 0.7) (layer B.Cu) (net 15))
 (segment (start 112.670001 77.745001) (end 116.205 81.28) (width 0.7) (layer B.Cu) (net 15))
 (segment (start 116.205 81.28) (end 116.205 85.725) (width 0.7) (layer B.Cu) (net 15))
 (segment (start 98.425 59.055) (end 92.075 59.055) (width 0.7) (layer B.Cu) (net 36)))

